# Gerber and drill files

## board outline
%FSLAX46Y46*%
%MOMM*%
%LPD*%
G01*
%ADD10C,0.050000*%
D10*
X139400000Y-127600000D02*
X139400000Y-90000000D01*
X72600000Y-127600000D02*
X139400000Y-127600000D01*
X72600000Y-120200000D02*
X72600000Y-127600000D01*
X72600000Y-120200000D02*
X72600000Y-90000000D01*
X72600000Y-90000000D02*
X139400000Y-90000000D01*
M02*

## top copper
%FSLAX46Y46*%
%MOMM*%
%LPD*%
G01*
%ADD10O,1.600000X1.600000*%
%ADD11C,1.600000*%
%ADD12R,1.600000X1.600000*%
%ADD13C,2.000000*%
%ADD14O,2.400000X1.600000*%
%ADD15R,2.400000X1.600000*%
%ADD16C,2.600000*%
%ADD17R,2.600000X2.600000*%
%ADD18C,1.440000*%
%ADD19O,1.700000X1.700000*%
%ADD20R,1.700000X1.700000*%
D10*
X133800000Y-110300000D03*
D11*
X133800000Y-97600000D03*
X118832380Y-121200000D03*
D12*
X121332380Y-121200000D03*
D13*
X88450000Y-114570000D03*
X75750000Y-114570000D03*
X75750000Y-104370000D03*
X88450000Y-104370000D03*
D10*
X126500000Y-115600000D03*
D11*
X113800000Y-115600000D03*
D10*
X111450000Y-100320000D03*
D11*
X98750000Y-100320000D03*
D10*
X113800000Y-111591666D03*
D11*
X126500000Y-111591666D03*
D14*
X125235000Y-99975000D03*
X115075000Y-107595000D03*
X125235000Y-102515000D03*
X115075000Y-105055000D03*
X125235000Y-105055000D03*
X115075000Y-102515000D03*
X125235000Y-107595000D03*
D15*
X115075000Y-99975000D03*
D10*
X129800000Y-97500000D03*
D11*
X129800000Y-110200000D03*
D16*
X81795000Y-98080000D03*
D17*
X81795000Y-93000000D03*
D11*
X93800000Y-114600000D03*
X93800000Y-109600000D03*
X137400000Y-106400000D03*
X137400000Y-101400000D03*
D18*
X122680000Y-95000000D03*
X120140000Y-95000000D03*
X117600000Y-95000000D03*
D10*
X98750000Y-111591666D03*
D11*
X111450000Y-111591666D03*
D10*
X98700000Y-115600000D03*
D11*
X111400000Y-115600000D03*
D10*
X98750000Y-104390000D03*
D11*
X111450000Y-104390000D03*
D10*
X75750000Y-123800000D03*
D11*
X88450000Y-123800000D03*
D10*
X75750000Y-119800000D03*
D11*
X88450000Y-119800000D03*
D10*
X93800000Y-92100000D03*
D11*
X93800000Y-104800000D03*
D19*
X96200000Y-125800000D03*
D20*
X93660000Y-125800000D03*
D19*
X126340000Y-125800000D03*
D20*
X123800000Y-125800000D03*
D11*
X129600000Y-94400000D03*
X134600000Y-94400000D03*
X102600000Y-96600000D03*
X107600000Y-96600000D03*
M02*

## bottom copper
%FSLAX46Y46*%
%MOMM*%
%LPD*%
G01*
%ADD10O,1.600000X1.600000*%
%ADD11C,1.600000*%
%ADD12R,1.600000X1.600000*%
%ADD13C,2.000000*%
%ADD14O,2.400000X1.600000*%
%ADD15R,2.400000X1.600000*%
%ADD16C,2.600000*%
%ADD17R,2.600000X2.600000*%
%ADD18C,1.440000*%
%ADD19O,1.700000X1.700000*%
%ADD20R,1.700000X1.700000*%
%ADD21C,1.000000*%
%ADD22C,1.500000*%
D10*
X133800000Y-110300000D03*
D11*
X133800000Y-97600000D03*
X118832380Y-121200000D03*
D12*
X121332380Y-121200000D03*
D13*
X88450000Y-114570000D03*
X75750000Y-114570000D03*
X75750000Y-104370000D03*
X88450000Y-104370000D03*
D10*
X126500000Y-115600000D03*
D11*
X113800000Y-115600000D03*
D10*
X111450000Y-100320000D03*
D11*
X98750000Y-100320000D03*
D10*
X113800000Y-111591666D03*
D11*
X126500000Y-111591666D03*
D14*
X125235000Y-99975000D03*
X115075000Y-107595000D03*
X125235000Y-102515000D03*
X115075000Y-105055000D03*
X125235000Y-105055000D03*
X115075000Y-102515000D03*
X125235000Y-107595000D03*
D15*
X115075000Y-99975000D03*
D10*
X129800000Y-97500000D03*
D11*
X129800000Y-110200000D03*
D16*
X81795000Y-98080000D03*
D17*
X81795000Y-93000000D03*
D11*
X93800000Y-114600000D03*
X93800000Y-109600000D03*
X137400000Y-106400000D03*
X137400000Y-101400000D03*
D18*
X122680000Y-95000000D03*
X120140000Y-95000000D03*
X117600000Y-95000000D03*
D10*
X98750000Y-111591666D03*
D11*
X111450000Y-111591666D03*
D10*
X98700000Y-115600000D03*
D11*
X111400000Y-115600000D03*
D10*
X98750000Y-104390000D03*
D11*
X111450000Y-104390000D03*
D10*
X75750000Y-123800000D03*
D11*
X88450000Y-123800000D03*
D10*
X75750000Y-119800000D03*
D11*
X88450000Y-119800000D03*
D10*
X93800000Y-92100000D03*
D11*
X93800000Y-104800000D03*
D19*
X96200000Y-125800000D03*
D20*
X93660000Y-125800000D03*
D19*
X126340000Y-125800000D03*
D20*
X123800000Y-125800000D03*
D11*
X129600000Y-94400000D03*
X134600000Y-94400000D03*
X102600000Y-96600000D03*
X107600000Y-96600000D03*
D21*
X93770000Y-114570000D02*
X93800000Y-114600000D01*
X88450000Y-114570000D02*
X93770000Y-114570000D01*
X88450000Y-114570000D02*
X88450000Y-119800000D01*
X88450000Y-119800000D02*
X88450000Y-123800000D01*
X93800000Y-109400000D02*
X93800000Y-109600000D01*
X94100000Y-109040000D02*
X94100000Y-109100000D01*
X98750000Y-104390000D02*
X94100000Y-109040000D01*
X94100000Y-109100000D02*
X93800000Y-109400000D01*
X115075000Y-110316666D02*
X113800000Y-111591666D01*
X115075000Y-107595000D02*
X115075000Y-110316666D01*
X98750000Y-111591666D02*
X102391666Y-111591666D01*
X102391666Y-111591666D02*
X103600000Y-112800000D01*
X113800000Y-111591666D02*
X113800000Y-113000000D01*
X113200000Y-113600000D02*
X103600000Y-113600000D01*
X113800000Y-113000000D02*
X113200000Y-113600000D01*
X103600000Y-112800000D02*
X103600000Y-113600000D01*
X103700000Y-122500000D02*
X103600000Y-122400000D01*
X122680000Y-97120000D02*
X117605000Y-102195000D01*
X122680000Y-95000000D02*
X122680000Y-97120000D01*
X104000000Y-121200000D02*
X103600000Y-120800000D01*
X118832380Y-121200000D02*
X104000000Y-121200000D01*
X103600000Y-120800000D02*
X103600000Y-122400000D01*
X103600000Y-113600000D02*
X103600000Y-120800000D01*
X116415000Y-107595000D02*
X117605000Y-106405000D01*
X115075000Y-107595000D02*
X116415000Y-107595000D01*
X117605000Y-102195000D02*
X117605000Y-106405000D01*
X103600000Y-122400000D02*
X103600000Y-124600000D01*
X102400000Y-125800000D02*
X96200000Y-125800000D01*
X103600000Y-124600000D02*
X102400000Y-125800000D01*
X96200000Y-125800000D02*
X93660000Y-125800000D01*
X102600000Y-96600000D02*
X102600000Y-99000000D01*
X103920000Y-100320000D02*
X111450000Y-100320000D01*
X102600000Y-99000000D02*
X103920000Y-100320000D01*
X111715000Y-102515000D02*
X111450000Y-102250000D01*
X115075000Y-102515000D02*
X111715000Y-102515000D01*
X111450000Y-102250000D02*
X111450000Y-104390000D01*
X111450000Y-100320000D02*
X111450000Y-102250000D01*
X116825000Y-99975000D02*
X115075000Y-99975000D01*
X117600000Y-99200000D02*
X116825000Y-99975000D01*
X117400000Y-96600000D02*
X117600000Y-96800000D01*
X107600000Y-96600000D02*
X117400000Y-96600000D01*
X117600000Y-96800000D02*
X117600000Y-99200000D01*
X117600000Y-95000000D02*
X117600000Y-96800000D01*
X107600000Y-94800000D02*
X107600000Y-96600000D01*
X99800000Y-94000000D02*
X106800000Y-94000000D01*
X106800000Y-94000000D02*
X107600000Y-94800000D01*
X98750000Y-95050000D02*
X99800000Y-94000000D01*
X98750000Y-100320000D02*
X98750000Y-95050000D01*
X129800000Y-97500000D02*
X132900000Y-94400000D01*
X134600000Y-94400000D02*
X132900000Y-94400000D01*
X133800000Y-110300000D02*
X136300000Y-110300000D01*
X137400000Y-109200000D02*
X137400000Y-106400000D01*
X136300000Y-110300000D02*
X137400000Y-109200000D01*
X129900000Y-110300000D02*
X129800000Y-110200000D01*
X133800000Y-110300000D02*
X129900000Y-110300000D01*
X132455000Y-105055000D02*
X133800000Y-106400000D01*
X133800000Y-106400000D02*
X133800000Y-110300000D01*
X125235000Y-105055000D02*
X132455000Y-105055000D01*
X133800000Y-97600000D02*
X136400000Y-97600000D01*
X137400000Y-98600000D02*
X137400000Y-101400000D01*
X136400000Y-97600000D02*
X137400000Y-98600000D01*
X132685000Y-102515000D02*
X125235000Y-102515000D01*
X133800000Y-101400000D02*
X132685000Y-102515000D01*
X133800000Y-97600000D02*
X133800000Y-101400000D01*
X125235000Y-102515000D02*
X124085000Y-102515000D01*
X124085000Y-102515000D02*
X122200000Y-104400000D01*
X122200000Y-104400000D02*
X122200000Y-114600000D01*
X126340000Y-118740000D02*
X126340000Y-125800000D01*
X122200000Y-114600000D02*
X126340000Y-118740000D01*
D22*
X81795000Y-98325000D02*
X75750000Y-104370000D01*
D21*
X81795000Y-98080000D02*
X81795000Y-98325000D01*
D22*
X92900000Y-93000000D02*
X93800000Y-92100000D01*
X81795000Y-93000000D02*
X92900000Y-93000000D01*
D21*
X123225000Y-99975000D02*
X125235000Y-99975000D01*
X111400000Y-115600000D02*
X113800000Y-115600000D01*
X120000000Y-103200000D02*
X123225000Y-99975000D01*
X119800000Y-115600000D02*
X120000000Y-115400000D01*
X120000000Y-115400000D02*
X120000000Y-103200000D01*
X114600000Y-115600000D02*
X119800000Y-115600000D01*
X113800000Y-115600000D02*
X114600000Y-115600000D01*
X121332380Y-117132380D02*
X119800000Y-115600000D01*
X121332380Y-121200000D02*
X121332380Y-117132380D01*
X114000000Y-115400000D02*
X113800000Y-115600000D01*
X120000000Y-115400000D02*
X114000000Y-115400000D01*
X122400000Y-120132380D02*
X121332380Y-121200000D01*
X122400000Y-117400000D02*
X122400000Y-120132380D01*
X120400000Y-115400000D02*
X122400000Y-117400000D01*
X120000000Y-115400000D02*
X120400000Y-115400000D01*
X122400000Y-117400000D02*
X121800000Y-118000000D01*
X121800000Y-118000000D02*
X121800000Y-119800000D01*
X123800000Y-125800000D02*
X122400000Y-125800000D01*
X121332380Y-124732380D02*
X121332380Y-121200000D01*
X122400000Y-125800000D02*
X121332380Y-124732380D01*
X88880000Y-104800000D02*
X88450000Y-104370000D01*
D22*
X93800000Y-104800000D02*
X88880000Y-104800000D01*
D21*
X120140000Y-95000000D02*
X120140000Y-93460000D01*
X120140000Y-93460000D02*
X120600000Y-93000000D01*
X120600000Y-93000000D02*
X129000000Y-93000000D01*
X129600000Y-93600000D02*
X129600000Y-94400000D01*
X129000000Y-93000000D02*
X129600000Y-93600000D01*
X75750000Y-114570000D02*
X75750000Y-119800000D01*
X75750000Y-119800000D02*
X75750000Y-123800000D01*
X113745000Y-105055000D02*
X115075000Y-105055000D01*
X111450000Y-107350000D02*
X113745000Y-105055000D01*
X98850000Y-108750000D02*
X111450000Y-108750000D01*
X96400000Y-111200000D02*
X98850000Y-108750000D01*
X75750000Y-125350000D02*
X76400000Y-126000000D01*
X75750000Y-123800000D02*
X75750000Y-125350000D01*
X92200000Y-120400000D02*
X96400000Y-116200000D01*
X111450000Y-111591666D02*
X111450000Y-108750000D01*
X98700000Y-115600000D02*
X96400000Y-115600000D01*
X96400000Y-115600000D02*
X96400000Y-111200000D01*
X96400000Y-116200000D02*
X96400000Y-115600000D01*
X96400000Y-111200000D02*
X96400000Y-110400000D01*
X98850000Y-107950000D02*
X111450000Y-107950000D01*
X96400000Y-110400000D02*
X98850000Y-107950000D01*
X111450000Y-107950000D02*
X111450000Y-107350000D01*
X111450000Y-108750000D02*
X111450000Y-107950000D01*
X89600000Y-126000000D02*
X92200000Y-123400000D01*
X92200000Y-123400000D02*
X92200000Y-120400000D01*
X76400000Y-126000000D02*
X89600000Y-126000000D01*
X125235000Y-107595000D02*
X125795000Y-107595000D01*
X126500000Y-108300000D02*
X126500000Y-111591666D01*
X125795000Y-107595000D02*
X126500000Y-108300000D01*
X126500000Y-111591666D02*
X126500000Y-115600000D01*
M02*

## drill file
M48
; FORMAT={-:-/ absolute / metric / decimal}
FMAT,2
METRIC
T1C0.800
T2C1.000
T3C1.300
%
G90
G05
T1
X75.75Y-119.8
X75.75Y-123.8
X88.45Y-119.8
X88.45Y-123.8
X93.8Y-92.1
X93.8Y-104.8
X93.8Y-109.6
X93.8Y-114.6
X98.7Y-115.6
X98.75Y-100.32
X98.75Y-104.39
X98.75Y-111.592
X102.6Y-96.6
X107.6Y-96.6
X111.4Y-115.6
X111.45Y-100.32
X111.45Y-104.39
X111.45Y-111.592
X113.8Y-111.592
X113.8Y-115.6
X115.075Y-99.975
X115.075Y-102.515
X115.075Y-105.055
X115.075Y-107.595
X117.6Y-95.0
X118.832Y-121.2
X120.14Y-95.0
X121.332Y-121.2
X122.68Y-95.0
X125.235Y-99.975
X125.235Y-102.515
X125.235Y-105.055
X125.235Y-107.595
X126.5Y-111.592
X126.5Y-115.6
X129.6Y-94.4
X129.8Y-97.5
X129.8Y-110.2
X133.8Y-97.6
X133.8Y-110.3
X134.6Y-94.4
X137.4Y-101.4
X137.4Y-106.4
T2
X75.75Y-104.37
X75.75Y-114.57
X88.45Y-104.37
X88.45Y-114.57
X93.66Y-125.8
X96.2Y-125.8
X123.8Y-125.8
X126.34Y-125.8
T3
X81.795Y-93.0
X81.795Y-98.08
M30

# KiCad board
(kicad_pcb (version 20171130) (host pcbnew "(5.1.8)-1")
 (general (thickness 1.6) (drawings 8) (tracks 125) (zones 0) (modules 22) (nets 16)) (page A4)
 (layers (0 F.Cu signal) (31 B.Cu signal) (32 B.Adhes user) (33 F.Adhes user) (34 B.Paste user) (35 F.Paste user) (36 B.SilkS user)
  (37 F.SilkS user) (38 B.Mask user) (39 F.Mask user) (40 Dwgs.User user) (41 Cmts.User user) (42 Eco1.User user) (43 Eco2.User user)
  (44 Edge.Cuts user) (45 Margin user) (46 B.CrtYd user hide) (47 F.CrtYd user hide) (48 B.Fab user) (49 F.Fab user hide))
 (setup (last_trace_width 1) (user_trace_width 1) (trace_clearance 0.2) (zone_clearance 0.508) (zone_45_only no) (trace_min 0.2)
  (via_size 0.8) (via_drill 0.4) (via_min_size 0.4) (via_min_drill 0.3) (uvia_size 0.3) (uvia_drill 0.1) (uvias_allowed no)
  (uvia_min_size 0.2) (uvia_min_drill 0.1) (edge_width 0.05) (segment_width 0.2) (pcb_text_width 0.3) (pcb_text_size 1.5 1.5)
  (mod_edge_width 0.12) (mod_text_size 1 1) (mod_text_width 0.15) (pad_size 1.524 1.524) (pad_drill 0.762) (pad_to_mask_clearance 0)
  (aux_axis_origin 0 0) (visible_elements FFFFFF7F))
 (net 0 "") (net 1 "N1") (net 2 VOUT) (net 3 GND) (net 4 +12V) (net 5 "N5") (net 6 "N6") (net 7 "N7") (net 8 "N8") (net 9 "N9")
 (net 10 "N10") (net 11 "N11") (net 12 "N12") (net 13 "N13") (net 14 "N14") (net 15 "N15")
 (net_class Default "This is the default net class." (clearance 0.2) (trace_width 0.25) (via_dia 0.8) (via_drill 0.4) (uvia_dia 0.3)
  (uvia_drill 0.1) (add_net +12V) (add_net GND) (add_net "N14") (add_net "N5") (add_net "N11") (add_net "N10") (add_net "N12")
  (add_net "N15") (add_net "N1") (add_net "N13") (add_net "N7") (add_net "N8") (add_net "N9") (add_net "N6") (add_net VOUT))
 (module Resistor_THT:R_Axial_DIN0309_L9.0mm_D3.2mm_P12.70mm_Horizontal (layer F.Cu) (at 133.8 97.6 270)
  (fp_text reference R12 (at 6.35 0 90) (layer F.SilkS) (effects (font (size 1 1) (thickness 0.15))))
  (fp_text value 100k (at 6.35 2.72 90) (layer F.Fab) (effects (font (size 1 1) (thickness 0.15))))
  (pad 2 thru_hole oval (at 12.7 0 270) (size 1.6 1.6) (drill 0.8) (layers *.Cu *.Mask) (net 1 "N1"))
  (pad 1 thru_hole circle (at 0 0 270) (size 1.6 1.6) (drill 0.8) (layers *.Cu *.Mask) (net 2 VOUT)))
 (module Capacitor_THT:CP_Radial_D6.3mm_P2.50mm (layer F.Cu) (at 121.33238 121.2 180)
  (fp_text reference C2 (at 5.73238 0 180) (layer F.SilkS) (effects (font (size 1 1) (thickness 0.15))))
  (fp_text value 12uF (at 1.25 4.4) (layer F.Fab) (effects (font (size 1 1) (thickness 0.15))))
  (pad 2 thru_hole circle (at 2.5 0 180) (size 1.6 1.6) (drill 0.8) (layers *.Cu *.Mask) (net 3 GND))
  (pad 1 thru_hole rect (at 0 0 180) (size 1.6 1.6) (drill 0.8) (layers *.Cu *.Mask) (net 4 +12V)))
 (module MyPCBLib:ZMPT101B (layer F.Cu) (at 82.1 109.45 270)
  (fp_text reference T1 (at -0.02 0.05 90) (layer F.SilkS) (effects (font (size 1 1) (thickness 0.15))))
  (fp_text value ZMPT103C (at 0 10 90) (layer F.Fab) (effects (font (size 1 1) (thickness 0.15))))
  (pad 4 thru_hole circle (at 5.12 -6.35 270) (size 2 2) (drill 1) (layers *.Cu *.Mask) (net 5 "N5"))
  (pad 3 thru_hole circle (at 5.12 6.35 270) (size 2 2) (drill 1) (layers *.Cu *.Mask) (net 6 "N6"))
  (pad 2 thru_hole circle (at -5.08 6.35 270) (size 2 2) (drill 1) (layers *.Cu *.Mask) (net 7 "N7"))
  (pad 1 thru_hole circle (at -5.08 -6.35 270) (size 2 2) (drill 1) (layers *.Cu *.Mask) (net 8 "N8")))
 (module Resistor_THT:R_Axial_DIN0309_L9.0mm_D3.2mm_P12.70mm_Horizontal (layer F.Cu) (at 113.8 115.6)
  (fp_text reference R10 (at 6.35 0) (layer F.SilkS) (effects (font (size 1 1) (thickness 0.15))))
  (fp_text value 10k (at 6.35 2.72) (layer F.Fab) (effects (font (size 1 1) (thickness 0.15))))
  (pad 2 thru_hole oval (at 12.7 0) (size 1.6 1.6) (drill 0.8) (layers *.Cu *.Mask) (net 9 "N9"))
  (pad 1 thru_hole circle (at 0 0) (size 1.6 1.6) (drill 0.8) (layers *.Cu *.Mask) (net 4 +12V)))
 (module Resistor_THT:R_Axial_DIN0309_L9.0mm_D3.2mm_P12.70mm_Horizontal (layer F.Cu) (at 98.75 100.32)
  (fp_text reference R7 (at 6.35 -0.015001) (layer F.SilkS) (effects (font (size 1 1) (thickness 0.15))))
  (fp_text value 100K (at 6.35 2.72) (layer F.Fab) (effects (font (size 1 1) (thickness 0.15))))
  (pad 2 thru_hole oval (at 12.7 0) (size 1.6 1.6) (drill 0.8) (layers *.Cu *.Mask) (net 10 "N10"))
  (pad 1 thru_hole circle (at 0 0) (size 1.6 1.6) (drill 0.8) (layers *.Cu *.Mask) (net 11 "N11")))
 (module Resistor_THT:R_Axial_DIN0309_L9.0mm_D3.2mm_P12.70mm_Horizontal (layer F.Cu) (at 126.5 111.591666 180)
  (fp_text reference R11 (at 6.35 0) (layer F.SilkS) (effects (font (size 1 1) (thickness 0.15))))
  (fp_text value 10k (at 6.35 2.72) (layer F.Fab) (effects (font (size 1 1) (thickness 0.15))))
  (pad 2 thru_hole oval (at 12.7 0 180) (size 1.6 1.6) (drill 0.8) (layers *.Cu *.Mask) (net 3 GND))
  (pad 1 thru_hole circle (at 0 0 180) (size 1.6 1.6) (drill 0.8) (layers *.Cu *.Mask) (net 9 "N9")))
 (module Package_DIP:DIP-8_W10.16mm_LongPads (layer F.Cu) (at 115.075 99.975)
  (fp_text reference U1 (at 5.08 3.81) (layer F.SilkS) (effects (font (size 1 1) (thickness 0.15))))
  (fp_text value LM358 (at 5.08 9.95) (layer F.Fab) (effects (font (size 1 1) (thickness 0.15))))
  (pad 8 thru_hole oval (at 10.16 0) (size 2.4 1.6) (drill 0.8) (layers *.Cu *.Mask) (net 4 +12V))
  (pad 4 thru_hole oval (at 0 7.62) (size 2.4 1.6) (drill 0.8) (layers *.Cu *.Mask) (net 3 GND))
  (pad 7 thru_hole oval (at 10.16 2.54) (size 2.4 1.6) (drill 0.8) (layers *.Cu *.Mask) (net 2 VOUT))
  (pad 3 thru_hole oval (at 0 5.08) (size 2.4 1.6) (drill 0.8) (layers *.Cu *.Mask) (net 6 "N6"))
  (pad 6 thru_hole oval (at 10.16 5.08) (size 2.4 1.6) (drill 0.8) (layers *.Cu *.Mask) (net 1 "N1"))
  (pad 2 thru_hole oval (at 0 2.54) (size 2.4 1.6) (drill 0.8) (layers *.Cu *.Mask) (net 10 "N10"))
  (pad 5 thru_hole oval (at 10.16 7.62) (size 2.4 1.6) (drill 0.8) (layers *.Cu *.Mask) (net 9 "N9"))
  (pad 1 thru_hole rect (at 0 0) (size 2.4 1.6) (drill 0.8) (layers *.Cu *.Mask) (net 11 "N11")))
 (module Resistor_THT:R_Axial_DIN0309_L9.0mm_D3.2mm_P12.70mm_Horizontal (layer F.Cu) (at 129.8 110.2 90)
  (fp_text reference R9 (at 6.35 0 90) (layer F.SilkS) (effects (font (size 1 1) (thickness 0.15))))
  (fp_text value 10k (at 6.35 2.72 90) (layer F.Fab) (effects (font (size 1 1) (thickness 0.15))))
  (pad 2 thru_hole oval (at 12.7 0 90) (size 1.6 1.6) (drill 0.8) (layers *.Cu *.Mask) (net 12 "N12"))
  (pad 1 thru_hole circle (at 0 0 90) (size 1.6 1.6) (drill 0.8) (layers *.Cu *.Mask) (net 1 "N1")))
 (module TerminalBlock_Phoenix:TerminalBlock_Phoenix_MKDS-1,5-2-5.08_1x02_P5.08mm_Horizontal (layer F.Cu) (at 81.795 93 270)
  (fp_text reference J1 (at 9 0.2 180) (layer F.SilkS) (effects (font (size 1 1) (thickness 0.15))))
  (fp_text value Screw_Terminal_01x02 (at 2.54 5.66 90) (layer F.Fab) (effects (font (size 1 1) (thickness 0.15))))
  (pad 2 thru_hole circle (at 5.08 0 270) (size 2.6 2.6) (drill 1.3) (layers *.Cu *.Mask) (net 7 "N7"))
  (pad 1 thru_hole rect (at 0 0 270) (size 2.6 2.6) (drill 1.3) (layers *.Cu *.Mask) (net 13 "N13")))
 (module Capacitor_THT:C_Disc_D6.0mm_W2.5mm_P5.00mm (layer F.Cu) (at 93.8 109.6 270)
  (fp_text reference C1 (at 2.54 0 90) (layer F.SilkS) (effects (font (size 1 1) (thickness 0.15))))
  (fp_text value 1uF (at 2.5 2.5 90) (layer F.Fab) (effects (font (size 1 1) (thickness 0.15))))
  (pad 2 thru_hole circle (at 5 0 270) (size 1.6 1.6) (drill 0.8) (layers *.Cu *.Mask) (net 5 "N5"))
  (pad 1 thru_hole circle (at 0 0 270) (size 1.6 1.6) (drill 0.8) (layers *.Cu *.Mask) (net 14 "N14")))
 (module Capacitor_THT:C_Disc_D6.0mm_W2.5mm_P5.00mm (layer F.Cu) (at 137.4 101.4 270)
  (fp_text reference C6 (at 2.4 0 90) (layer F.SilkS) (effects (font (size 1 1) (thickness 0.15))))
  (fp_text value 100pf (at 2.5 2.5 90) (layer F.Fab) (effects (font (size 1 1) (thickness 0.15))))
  (pad 2 thru_hole circle (at 5 0 270) (size 1.6 1.6) (drill 0.8) (layers *.Cu *.Mask) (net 1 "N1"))
  (pad 1 thru_hole circle (at 0 0 270) (size 1.6 1.6) (drill 0.8) (layers *.Cu *.Mask) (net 2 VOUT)))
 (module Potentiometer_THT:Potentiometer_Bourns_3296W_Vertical (layer F.Cu) (at 117.6 95 180)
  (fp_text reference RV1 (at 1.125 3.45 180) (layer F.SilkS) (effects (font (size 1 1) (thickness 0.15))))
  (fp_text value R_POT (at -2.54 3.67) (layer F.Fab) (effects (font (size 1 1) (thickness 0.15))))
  (pad 3 thru_hole circle (at -5.08 0 180) (size 1.44 1.44) (drill 0.8) (layers *.Cu *.Mask) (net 3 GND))
  (pad 2 thru_hole circle (at -2.54 0 180) (size 1.44 1.44) (drill 0.8) (layers *.Cu *.Mask) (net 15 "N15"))
  (pad 1 thru_hole circle (at 0 0 180) (size 1.44 1.44) (drill 0.8) (layers *.Cu *.Mask) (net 11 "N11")))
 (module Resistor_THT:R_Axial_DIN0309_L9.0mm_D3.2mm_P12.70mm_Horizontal (layer F.Cu) (at 111.45 111.591666 180)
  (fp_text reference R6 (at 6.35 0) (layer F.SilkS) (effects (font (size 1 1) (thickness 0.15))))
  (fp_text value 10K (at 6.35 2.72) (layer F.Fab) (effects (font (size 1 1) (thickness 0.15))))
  (pad 2 thru_hole oval (at 12.7 0 180) (size 1.6 1.6) (drill 0.8) (layers *.Cu *.Mask) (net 3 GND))
  (pad 1 thru_hole circle (at 0 0 180) (size 1.6 1.6) (drill 0.8) (layers *.Cu *.Mask) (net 6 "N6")))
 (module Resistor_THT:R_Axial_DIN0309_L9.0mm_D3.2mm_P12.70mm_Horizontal (layer F.Cu) (at 111.4 115.6 180)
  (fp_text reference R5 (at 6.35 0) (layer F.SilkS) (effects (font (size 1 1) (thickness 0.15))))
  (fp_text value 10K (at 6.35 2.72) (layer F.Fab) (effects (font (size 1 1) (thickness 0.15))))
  (pad 2 thru_hole oval (at 12.7 0 180) (size 1.6 1.6) (drill 0.8) (layers *.Cu *.Mask) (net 6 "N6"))
  (pad 1 thru_hole circle (at 0 0 180) (size 1.6 1.6) (drill 0.8) (layers *.Cu *.Mask) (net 4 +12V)))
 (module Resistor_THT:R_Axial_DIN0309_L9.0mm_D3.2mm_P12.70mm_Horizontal (layer F.Cu) (at 111.45 104.39 180)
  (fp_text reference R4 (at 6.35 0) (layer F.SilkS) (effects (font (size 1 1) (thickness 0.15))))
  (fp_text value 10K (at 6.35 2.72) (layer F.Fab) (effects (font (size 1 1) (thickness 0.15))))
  (pad 2 thru_hole oval (at 12.7 0 180) (size 1.6 1.6) (drill 0.8) (layers *.Cu *.Mask) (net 14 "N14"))
  (pad 1 thru_hole circle (at 0 0 180) (size 1.6 1.6) (drill 0.8) (layers *.Cu *.Mask) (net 10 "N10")))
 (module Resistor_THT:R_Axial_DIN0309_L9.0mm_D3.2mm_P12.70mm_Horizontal (layer F.Cu) (at 88.45 123.8 180)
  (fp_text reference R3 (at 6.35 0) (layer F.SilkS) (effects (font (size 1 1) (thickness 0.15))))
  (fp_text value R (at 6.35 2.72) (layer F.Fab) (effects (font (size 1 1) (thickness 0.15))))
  (pad 2 thru_hole oval (at 12.7 0 180) (size 1.6 1.6) (drill 0.8) (layers *.Cu *.Mask) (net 6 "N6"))
  (pad 1 thru_hole circle (at 0 0 180) (size 1.6 1.6) (drill 0.8) (layers *.Cu *.Mask) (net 5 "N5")))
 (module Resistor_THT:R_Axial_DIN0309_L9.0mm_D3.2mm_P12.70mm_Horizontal (layer F.Cu) (at 88.45 119.8 180)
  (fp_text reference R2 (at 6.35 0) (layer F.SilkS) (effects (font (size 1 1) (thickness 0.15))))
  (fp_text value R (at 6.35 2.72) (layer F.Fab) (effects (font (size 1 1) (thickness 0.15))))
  (pad 2 thru_hole oval (at 12.7 0 180) (size 1.6 1.6) (drill 0.8) (layers *.Cu *.Mask) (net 6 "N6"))
  (pad 1 thru_hole circle (at 0 0 180) (size 1.6 1.6) (drill 0.8) (layers *.Cu *.Mask) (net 5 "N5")))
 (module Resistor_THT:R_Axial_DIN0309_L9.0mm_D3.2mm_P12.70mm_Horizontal (layer F.Cu) (at 93.8 104.8 90)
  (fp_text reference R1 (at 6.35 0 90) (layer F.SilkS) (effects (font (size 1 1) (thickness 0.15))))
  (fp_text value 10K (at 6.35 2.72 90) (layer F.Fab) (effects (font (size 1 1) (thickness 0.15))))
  (pad 2 thru_hole oval (at 12.7 0 90) (size 1.6 1.6) (drill 0.8) (layers *.Cu *.Mask) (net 13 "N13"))
  (pad 1 thru_hole circle (at 0 0 90) (size 1.6 1.6) (drill 0.8) (layers *.Cu *.Mask) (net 8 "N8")))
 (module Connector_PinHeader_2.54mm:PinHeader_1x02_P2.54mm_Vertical (layer F.Cu) (at 93.66 125.8 90)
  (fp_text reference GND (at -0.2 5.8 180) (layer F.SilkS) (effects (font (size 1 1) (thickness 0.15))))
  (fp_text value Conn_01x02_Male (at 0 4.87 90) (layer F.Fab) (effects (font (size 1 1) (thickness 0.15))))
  (pad 2 thru_hole oval (at 0 2.54 90) (size 1.7 1.7) (drill 1) (layers *.Cu *.Mask) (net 3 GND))
  (pad 1 thru_hole rect (at 0 0 90) (size 1.7 1.7) (drill 1) (layers *.Cu *.Mask) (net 3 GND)))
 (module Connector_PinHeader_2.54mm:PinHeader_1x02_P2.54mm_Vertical (layer F.Cu) (at 123.8 125.8 90)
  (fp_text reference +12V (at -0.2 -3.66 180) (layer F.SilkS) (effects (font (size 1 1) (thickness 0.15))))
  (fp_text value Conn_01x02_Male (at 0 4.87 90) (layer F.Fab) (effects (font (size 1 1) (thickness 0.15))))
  (pad 2 thru_hole oval (at 0 2.54 90) (size 1.7 1.7) (drill 1) (layers *.Cu *.Mask) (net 2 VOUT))
  (pad 1 thru_hole rect (at 0 0 90) (size 1.7 1.7) (drill 1) (layers *.Cu *.Mask) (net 4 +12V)))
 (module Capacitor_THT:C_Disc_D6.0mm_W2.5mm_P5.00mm (layer F.Cu) (at 134.6 94.4 180)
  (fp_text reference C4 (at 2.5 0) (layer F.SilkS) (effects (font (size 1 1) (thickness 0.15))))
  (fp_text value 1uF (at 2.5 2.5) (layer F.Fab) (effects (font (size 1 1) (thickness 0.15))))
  (pad 2 thru_hole circle (at 5 0 180) (size 1.6 1.6) (drill 0.8) (layers *.Cu *.Mask) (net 15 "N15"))
  (pad 1 thru_hole circle (at 0 0 180) (size 1.6 1.6) (drill 0.8) (layers *.Cu *.Mask) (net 12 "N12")))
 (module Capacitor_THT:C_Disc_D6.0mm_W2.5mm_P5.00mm (layer F.Cu) (at 107.6 96.6 180)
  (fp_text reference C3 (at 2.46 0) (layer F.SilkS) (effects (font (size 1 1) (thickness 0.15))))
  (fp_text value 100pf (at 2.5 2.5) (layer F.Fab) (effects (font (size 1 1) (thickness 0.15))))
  (pad 2 thru_hole circle (at 5 0 180) (size 1.6 1.6) (drill 0.8) (layers *.Cu *.Mask) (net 10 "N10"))
  (pad 1 thru_hole circle (at 0 0 180) (size 1.6 1.6) (drill 0.8) (layers *.Cu *.Mask) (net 11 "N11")))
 (gr_line (start 139.4 127.6) (end 139.4 90) (layer Edge.Cuts) (width 0.05))
 (gr_line (start 72.6 127.6) (end 139.4 127.6) (layer Edge.Cuts) (width 0.05))
 (gr_line (start 72.6 120.2) (end 72.6 127.6) (layer Edge.Cuts) (width 0.05))
 (gr_line (start 72.6 120.2) (end 72.6 90) (layer Edge.Cuts) (width 0.05))
 (gr_line (start 72.6 90) (end 139.4 90) (layer Edge.Cuts) (width 0.05))
 (segment (start 93.77 114.57) (end 93.8 114.6) (width 1) (layer B.Cu) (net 5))
 (segment (start 88.45 114.57) (end 93.77 114.57) (width 1) (layer B.Cu) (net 5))
 (segment (start 88.45 114.57) (end 88.45 119.8) (width 1) (layer B.Cu) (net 5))
 (segment (start 88.45 119.8) (end 88.45 123.8) (width 1) (layer B.Cu) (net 5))
 (segment (start 93.8 109.4) (end 93.8 109.6) (width 1) (layer B.Cu) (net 14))
 (segment (start 94.1 109.04) (end 94.1 109.1) (width 1) (layer B.Cu) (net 14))
 (segment (start 98.75 104.39) (end 94.1 109.04) (width 1) (layer B.Cu) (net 14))
 (segment (start 94.1 109.1) (end 93.8 109.4) (width 1) (layer B.Cu) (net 14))
 (segment (start 115.075 110.316666) (end 113.8 111.591666) (width 1) (layer B.Cu) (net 3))
 (segment (start 115.075 107.595) (end 115.075 110.316666) (width 1) (layer B.Cu) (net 3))
 (segment (start 98.75 111.591666) (end 102.391666 111.591666) (width 1) (layer B.Cu) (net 3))
 (segment (start 102.391666 111.591666) (end 103.6 112.8) (width 1) (layer B.Cu) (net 3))
 (segment (start 113.8 111.591666) (end 113.8 113) (width 1) (layer B.Cu) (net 3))
 (segment (start 113.2 113.6) (end 103.6 113.6) (width 1) (layer B.Cu) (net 3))
 (segment (start 113.8 113) (end 113.2 113.6) (width 1) (layer B.Cu) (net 3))
 (segment (start 103.6 112.8) (end 103.6 113.6) (width 1) (layer B.Cu) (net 3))
 (segment (start 103.7 122.5) (end 103.6 122.4) (width 1) (layer B.Cu) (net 3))
 (segment (start 122.68 97.12) (end 117.605 102.195) (width 1) (layer B.Cu) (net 3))
 (segment (start 122.68 95) (end 122.68 97.12) (width 1) (layer B.Cu) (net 3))
 (segment (start 104 121.2) (end 103.6 120.8) (width 1) (layer B.Cu) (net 3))
 (segment (start 118.83238 121.2) (end 104 121.2) (width 1) (layer B.Cu) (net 3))
 (segment (start 103.6 120.8) (end 103.6 122.4) (width 1) (layer B.Cu) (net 3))
 (segment (start 103.6 113.6) (end 103.6 120.8) (width 1) (layer B.Cu) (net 3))
 (segment (start 116.415 107.595) (end 117.605 106.405) (width 1) (layer B.Cu) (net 3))
 (segment (start 115.075 107.595) (end 116.415 107.595) (width 1) (layer B.Cu) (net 3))
 (segment (start 117.605 102.195) (end 117.605 106.405) (width 1) (layer B.Cu) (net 3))
 (segment (start 103.6 122.4) (end 103.6 124.6) (width 1) (layer B.Cu) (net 3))
 (segment (start 102.4 125.8) (end 96.2 125.8) (width 1) (layer B.Cu) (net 3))
 (segment (start 103.6 124.6) (end 102.4 125.8) (width 1) (layer B.Cu) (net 3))
 (segment (start 96.2 125.8) (end 93.66 125.8) (width 1) (layer B.Cu) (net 3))
 (segment (start 102.6 96.6) (end 102.6 99) (width 1) (layer B.Cu) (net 10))
 (segment (start 103.92 100.32) (end 111.45 100.32) (width 1) (layer B.Cu) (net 10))
 (segment (start 102.6 99) (end 103.92 100.32) (width 1) (layer B.Cu) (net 10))
 (segment (start 111.715 102.515) (end 111.45 102.25) (width 1) (layer B.Cu) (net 10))
 (segment (start 115.075 102.515) (end 111.715 102.515) (width 1) (layer B.Cu) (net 10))
 (segment (start 111.45 102.25) (end 111.45 104.39) (width 1) (layer B.Cu) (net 10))
 (segment (start 111.45 100.32) (end 111.45 102.25) (width 1) (layer B.Cu) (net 10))
 (segment (start 116.825 99.975) (end 115.075 99.975) (width 1) (layer B.Cu) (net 11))
 (segment (start 117.6 99.2) (end 116.825 99.975) (width 1) (layer B.Cu) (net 11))
 (segment (start 117.4 96.6) (end 117.6 96.8) (width 1) (layer B.Cu) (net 11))
 (segment (start 107.6 96.6) (end 117.4 96.6) (width 1) (layer B.Cu) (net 11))
 (segment (start 117.6 96.8) (end 117.6 99.2) (width 1) (layer B.Cu) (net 11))
 (segment (start 117.6 95) (end 117.6 96.8) (width 1) (layer B.Cu) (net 11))
 (segment (start 107.6 94.8) (end 107.6 96.6) (width 1) (layer B.Cu) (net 11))
 (segment (start 99.8 94) (end 106.8 94) (width 1) (layer B.Cu) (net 11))
 (segment (start 106.8 94) (end 107.6 94.8) (width 1) (layer B.Cu) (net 11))
 (segment (start 98.75 95.05) (end 99.8 94) (width 1) (layer B.Cu) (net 11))
 (segment (start 98.75 100.32) (end 98.75 95.05) (width 1) (layer B.Cu) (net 11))
 (segment (start 129.8 97.5) (end 132.9 94.4) (width 1) (layer B.Cu) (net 12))
 (segment (start 134.6 94.4) (end 132.9 94.4) (width 1) (layer B.Cu) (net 12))
 (segment (start 133.8 110.3) (end 136.3 110.3) (width 1) (layer B.Cu) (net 1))
 (segment (start 137.4 109.2) (end 137.4 106.4) (width 1) (layer B.Cu) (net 1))
 (segment (start 136.3 110.3) (end 137.4 109.2) (width 1) (layer B.Cu) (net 1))
 (segment (start 129.9 110.3) (end 129.8 110.2) (width 1) (layer B.Cu) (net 1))
 (segment (start 133.8 110.3) (end 129.9 110.3) (width 1) (layer B.Cu) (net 1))
 (segment (start 132.455 105.055) (end 133.8 106.4) (width 1) (layer B.Cu) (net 1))
 (segment (start 133.8 106.4) (end 133.8 110.3) (width 1) (layer B.Cu) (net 1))
 (segment (start 125.235 105.055) (end 132.455 105.055) (width 1) (layer B.Cu) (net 1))
 (segment (start 133.8 97.6) (end 136.4 97.6) (width 1) (layer B.Cu) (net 2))
 (segment (start 137.4 98.6) (end 137.4 101.4) (width 1) (layer B.Cu) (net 2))
 (segment (start 136.4 97.6) (end 137.4 98.6) (width 1) (layer B.Cu) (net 2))
 (segment (start 132.685 102.515) (end 125.235 102.515) (width 1) (layer B.Cu) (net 2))
 (segment (start 133.8 101.4) (end 132.685 102.515) (width 1) (layer B.Cu) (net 2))
 (segment (start 133.8 97.6) (end 133.8 101.4) (width 1) (layer B.Cu) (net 2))
 (segment (start 125.235 102.515) (end 124.085 102.515) (width 1) (layer B.Cu) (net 2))
 (segment (start 124.085 102.515) (end 122.2 104.4) (width 1) (layer B.Cu) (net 2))
 (segment (start 122.2 104.4) (end 122.2 114.6) (width 1) (layer B.Cu) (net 2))
 (segment (start 126.34 118.74) (end 126.34 125.8) (width 1) (layer B.Cu) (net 2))
 (segment (start 122.2 114.6) (end 126.34 118.74) (width 1) (layer B.Cu) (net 2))
 (segment (start 81.795 98.325) (end 75.75 104.37) (width 1.5) (layer B.Cu) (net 7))
 (segment (start 81.795 98.08) (end 81.795 98.325) (width 1) (layer B.Cu) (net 7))
 (segment (start 92.9 93) (end 93.8 92.1) (width 1.5) (layer B.Cu) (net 13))
 (segment (start 81.795 93) (end 92.9 93) (width 1.5) (layer B.Cu) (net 13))
 (segment (start 123.225 99.975) (end 125.235 99.975) (width 1) (layer B.Cu) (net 4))
 (segment (start 111.4 115.6) (end 113.8 115.6) (width 1) (layer B.Cu) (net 4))
 (segment (start 120 103.2) (end 123.225 99.975) (width 1) (layer B.Cu) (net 4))
 (segment (start 119.8 115.6) (end 120 115.4) (width 1) (layer B.Cu) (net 4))
 (segment (start 120 115.4) (end 120 103.2) (width 1) (layer B.Cu) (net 4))
 (segment (start 114.6 115.6) (end 119.8 115.6) (width 1) (layer B.Cu) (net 4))
 (segment (start 113.8 115.6) (end 114.6 115.6) (width 1) (layer B.Cu) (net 4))
 (segment (start 121.33238 117.13238) (end 119.8 115.6) (width 1) (layer B.Cu) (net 4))
 (segment (start 121.33238 121.2) (end 121.33238 117.13238) (width 1) (layer B.Cu) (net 4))
 (segment (start 114 115.4) (end 113.8 115.6) (width 1) (layer B.Cu) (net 4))
 (segment (start 120 115.4) (end 114 115.4) (width 1) (layer B.Cu) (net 4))
 (segment (start 122.4 120.13238) (end 121.33238 121.2) (width 1) (layer B.Cu) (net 4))
 (segment (start 122.4 117.4) (end 122.4 120.13238) (width 1) (layer B.Cu) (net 4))
 (segment (start 120.4 115.4) (end 122.4 117.4) (width 1) (layer B.Cu) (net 4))
 (segment (start 120 115.4) (end 120.4 115.4) (width 1) (layer B.Cu) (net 4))
 (segment (start 122.4 117.4) (end 121.8 118) (width 1) (layer B.Cu) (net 4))
 (segment (start 121.8 118) (end 121.8 119.8) (width 1) (layer B.Cu) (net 4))
 (segment (start 123.8 125.8) (end 122.4 125.8) (width 1) (layer B.Cu) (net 4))
 (segment (start 121.33238 124.73238) (end 121.33238 121.2) (width 1) (layer B.Cu) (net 4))
 (segment (start 122.4 125.8) (end 121.33238 124.73238) (width 1) (layer B.Cu) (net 4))
 (segment (start 88.88 104.8) (end 88.45 104.37) (width 1) (layer B.Cu) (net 8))
 (segment (start 93.8 104.8) (end 88.88 104.8) (width 1.5) (layer B.Cu) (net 8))
 (segment (start 120.14 95) (end 120.14 93.46) (width 1) (layer B.Cu) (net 15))
 (segment (start 120.14 93.46) (end 120.6 93) (width 1) (layer B.Cu) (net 15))
 (segment (start 120.6 93) (end 129 93) (width 1) (layer B.Cu) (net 15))
 (segment (start 129.6 93.6) (end 129.6 94.4) (width 1) (layer B.Cu) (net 15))
 (segment (start 129 93) (end 129.6 93.6) (width 1) (layer B.Cu) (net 15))
 (segment (start 75.75 114.57) (end 75.75 119.8) (width 1) (layer B.Cu) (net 6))
 (segment (start 75.75 119.8) (end 75.75 123.8) (width 1) (layer B.Cu) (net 6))
 (segment (start 113.745 105.055) (end 115.075 105.055) (width 1) (layer B.Cu) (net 6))
 (segment (start 111.45 107.35) (end 113.745 105.055) (width 1) (layer B.Cu) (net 6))
 (segment (start 98.85 108.75) (end 111.45 108.75) (width 1) (layer B.Cu) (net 6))
 (segment (start 96.4 111.2) (end 98.85 108.75) (width 1) (layer B.Cu) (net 6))
 (segment (start 75.75 125.35) (end 76.4 126) (width 1) (layer B.Cu) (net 6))
 (segment (start 75.75 123.8) (end 75.75 125.35) (width 1) (layer B.Cu) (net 6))
 (segment (start 92.2 120.4) (end 96.4 116.2) (width 1) (layer B.Cu) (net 6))
 (segment (start 111.45 111.591666) (end 111.45 108.75) (width 1) (layer B.Cu) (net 6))
 (segment (start 98.7 115.6) (end 96.4 115.6) (width 1) (layer B.Cu) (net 6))
 (segment (start 96.4 115.6) (end 96.4 111.2) (width 1) (layer B.Cu) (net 6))
 (segment (start 96.4 116.2) (end 96.4 115.6) (width 1) (layer B.Cu) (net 6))
 (segment (start 96.4 111.2) (end 96.4 110.4) (width 1) (layer B.Cu) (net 6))
 (segment (start 98.85 107.95) (end 111.45 107.95) (width 1) (layer B.Cu) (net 6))
 (segment (start 96.4 110.4) (end 98.85 107.95) (width 1) (layer B.Cu) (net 6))
 (segment (start 111.45 107.95) (end 111.45 107.35) (width 1) (layer B.Cu) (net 6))
 (segment (start 111.45 108.75) (end 111.45 107.95) (width 1) (layer B.Cu) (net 6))
 (segment (start 89.6 126) (end 92.2 123.4) (width 1) (layer B.Cu) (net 6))
 (segment (start 92.2 123.4) (end 92.2 120.4) (width 1) (layer B.Cu) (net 6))
 (segment (start 76.4 126) (end 89.6 126) (width 1) (layer B.Cu) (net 6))
 (segment (start 125.235 107.595) (end 125.795 107.595) (width 1) (layer B.Cu) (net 9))
 (segment (start 126.5 108.3) (end 126.5 111.591666) (width 1) (layer B.Cu) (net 9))
 (segment (start 125.795 107.595) (end 126.5 108.3) (width 1) (layer B.Cu) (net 9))
 (segment (start 126.5 111.591666) (end 126.5 115.6) (width 1) (layer B.Cu) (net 9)))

